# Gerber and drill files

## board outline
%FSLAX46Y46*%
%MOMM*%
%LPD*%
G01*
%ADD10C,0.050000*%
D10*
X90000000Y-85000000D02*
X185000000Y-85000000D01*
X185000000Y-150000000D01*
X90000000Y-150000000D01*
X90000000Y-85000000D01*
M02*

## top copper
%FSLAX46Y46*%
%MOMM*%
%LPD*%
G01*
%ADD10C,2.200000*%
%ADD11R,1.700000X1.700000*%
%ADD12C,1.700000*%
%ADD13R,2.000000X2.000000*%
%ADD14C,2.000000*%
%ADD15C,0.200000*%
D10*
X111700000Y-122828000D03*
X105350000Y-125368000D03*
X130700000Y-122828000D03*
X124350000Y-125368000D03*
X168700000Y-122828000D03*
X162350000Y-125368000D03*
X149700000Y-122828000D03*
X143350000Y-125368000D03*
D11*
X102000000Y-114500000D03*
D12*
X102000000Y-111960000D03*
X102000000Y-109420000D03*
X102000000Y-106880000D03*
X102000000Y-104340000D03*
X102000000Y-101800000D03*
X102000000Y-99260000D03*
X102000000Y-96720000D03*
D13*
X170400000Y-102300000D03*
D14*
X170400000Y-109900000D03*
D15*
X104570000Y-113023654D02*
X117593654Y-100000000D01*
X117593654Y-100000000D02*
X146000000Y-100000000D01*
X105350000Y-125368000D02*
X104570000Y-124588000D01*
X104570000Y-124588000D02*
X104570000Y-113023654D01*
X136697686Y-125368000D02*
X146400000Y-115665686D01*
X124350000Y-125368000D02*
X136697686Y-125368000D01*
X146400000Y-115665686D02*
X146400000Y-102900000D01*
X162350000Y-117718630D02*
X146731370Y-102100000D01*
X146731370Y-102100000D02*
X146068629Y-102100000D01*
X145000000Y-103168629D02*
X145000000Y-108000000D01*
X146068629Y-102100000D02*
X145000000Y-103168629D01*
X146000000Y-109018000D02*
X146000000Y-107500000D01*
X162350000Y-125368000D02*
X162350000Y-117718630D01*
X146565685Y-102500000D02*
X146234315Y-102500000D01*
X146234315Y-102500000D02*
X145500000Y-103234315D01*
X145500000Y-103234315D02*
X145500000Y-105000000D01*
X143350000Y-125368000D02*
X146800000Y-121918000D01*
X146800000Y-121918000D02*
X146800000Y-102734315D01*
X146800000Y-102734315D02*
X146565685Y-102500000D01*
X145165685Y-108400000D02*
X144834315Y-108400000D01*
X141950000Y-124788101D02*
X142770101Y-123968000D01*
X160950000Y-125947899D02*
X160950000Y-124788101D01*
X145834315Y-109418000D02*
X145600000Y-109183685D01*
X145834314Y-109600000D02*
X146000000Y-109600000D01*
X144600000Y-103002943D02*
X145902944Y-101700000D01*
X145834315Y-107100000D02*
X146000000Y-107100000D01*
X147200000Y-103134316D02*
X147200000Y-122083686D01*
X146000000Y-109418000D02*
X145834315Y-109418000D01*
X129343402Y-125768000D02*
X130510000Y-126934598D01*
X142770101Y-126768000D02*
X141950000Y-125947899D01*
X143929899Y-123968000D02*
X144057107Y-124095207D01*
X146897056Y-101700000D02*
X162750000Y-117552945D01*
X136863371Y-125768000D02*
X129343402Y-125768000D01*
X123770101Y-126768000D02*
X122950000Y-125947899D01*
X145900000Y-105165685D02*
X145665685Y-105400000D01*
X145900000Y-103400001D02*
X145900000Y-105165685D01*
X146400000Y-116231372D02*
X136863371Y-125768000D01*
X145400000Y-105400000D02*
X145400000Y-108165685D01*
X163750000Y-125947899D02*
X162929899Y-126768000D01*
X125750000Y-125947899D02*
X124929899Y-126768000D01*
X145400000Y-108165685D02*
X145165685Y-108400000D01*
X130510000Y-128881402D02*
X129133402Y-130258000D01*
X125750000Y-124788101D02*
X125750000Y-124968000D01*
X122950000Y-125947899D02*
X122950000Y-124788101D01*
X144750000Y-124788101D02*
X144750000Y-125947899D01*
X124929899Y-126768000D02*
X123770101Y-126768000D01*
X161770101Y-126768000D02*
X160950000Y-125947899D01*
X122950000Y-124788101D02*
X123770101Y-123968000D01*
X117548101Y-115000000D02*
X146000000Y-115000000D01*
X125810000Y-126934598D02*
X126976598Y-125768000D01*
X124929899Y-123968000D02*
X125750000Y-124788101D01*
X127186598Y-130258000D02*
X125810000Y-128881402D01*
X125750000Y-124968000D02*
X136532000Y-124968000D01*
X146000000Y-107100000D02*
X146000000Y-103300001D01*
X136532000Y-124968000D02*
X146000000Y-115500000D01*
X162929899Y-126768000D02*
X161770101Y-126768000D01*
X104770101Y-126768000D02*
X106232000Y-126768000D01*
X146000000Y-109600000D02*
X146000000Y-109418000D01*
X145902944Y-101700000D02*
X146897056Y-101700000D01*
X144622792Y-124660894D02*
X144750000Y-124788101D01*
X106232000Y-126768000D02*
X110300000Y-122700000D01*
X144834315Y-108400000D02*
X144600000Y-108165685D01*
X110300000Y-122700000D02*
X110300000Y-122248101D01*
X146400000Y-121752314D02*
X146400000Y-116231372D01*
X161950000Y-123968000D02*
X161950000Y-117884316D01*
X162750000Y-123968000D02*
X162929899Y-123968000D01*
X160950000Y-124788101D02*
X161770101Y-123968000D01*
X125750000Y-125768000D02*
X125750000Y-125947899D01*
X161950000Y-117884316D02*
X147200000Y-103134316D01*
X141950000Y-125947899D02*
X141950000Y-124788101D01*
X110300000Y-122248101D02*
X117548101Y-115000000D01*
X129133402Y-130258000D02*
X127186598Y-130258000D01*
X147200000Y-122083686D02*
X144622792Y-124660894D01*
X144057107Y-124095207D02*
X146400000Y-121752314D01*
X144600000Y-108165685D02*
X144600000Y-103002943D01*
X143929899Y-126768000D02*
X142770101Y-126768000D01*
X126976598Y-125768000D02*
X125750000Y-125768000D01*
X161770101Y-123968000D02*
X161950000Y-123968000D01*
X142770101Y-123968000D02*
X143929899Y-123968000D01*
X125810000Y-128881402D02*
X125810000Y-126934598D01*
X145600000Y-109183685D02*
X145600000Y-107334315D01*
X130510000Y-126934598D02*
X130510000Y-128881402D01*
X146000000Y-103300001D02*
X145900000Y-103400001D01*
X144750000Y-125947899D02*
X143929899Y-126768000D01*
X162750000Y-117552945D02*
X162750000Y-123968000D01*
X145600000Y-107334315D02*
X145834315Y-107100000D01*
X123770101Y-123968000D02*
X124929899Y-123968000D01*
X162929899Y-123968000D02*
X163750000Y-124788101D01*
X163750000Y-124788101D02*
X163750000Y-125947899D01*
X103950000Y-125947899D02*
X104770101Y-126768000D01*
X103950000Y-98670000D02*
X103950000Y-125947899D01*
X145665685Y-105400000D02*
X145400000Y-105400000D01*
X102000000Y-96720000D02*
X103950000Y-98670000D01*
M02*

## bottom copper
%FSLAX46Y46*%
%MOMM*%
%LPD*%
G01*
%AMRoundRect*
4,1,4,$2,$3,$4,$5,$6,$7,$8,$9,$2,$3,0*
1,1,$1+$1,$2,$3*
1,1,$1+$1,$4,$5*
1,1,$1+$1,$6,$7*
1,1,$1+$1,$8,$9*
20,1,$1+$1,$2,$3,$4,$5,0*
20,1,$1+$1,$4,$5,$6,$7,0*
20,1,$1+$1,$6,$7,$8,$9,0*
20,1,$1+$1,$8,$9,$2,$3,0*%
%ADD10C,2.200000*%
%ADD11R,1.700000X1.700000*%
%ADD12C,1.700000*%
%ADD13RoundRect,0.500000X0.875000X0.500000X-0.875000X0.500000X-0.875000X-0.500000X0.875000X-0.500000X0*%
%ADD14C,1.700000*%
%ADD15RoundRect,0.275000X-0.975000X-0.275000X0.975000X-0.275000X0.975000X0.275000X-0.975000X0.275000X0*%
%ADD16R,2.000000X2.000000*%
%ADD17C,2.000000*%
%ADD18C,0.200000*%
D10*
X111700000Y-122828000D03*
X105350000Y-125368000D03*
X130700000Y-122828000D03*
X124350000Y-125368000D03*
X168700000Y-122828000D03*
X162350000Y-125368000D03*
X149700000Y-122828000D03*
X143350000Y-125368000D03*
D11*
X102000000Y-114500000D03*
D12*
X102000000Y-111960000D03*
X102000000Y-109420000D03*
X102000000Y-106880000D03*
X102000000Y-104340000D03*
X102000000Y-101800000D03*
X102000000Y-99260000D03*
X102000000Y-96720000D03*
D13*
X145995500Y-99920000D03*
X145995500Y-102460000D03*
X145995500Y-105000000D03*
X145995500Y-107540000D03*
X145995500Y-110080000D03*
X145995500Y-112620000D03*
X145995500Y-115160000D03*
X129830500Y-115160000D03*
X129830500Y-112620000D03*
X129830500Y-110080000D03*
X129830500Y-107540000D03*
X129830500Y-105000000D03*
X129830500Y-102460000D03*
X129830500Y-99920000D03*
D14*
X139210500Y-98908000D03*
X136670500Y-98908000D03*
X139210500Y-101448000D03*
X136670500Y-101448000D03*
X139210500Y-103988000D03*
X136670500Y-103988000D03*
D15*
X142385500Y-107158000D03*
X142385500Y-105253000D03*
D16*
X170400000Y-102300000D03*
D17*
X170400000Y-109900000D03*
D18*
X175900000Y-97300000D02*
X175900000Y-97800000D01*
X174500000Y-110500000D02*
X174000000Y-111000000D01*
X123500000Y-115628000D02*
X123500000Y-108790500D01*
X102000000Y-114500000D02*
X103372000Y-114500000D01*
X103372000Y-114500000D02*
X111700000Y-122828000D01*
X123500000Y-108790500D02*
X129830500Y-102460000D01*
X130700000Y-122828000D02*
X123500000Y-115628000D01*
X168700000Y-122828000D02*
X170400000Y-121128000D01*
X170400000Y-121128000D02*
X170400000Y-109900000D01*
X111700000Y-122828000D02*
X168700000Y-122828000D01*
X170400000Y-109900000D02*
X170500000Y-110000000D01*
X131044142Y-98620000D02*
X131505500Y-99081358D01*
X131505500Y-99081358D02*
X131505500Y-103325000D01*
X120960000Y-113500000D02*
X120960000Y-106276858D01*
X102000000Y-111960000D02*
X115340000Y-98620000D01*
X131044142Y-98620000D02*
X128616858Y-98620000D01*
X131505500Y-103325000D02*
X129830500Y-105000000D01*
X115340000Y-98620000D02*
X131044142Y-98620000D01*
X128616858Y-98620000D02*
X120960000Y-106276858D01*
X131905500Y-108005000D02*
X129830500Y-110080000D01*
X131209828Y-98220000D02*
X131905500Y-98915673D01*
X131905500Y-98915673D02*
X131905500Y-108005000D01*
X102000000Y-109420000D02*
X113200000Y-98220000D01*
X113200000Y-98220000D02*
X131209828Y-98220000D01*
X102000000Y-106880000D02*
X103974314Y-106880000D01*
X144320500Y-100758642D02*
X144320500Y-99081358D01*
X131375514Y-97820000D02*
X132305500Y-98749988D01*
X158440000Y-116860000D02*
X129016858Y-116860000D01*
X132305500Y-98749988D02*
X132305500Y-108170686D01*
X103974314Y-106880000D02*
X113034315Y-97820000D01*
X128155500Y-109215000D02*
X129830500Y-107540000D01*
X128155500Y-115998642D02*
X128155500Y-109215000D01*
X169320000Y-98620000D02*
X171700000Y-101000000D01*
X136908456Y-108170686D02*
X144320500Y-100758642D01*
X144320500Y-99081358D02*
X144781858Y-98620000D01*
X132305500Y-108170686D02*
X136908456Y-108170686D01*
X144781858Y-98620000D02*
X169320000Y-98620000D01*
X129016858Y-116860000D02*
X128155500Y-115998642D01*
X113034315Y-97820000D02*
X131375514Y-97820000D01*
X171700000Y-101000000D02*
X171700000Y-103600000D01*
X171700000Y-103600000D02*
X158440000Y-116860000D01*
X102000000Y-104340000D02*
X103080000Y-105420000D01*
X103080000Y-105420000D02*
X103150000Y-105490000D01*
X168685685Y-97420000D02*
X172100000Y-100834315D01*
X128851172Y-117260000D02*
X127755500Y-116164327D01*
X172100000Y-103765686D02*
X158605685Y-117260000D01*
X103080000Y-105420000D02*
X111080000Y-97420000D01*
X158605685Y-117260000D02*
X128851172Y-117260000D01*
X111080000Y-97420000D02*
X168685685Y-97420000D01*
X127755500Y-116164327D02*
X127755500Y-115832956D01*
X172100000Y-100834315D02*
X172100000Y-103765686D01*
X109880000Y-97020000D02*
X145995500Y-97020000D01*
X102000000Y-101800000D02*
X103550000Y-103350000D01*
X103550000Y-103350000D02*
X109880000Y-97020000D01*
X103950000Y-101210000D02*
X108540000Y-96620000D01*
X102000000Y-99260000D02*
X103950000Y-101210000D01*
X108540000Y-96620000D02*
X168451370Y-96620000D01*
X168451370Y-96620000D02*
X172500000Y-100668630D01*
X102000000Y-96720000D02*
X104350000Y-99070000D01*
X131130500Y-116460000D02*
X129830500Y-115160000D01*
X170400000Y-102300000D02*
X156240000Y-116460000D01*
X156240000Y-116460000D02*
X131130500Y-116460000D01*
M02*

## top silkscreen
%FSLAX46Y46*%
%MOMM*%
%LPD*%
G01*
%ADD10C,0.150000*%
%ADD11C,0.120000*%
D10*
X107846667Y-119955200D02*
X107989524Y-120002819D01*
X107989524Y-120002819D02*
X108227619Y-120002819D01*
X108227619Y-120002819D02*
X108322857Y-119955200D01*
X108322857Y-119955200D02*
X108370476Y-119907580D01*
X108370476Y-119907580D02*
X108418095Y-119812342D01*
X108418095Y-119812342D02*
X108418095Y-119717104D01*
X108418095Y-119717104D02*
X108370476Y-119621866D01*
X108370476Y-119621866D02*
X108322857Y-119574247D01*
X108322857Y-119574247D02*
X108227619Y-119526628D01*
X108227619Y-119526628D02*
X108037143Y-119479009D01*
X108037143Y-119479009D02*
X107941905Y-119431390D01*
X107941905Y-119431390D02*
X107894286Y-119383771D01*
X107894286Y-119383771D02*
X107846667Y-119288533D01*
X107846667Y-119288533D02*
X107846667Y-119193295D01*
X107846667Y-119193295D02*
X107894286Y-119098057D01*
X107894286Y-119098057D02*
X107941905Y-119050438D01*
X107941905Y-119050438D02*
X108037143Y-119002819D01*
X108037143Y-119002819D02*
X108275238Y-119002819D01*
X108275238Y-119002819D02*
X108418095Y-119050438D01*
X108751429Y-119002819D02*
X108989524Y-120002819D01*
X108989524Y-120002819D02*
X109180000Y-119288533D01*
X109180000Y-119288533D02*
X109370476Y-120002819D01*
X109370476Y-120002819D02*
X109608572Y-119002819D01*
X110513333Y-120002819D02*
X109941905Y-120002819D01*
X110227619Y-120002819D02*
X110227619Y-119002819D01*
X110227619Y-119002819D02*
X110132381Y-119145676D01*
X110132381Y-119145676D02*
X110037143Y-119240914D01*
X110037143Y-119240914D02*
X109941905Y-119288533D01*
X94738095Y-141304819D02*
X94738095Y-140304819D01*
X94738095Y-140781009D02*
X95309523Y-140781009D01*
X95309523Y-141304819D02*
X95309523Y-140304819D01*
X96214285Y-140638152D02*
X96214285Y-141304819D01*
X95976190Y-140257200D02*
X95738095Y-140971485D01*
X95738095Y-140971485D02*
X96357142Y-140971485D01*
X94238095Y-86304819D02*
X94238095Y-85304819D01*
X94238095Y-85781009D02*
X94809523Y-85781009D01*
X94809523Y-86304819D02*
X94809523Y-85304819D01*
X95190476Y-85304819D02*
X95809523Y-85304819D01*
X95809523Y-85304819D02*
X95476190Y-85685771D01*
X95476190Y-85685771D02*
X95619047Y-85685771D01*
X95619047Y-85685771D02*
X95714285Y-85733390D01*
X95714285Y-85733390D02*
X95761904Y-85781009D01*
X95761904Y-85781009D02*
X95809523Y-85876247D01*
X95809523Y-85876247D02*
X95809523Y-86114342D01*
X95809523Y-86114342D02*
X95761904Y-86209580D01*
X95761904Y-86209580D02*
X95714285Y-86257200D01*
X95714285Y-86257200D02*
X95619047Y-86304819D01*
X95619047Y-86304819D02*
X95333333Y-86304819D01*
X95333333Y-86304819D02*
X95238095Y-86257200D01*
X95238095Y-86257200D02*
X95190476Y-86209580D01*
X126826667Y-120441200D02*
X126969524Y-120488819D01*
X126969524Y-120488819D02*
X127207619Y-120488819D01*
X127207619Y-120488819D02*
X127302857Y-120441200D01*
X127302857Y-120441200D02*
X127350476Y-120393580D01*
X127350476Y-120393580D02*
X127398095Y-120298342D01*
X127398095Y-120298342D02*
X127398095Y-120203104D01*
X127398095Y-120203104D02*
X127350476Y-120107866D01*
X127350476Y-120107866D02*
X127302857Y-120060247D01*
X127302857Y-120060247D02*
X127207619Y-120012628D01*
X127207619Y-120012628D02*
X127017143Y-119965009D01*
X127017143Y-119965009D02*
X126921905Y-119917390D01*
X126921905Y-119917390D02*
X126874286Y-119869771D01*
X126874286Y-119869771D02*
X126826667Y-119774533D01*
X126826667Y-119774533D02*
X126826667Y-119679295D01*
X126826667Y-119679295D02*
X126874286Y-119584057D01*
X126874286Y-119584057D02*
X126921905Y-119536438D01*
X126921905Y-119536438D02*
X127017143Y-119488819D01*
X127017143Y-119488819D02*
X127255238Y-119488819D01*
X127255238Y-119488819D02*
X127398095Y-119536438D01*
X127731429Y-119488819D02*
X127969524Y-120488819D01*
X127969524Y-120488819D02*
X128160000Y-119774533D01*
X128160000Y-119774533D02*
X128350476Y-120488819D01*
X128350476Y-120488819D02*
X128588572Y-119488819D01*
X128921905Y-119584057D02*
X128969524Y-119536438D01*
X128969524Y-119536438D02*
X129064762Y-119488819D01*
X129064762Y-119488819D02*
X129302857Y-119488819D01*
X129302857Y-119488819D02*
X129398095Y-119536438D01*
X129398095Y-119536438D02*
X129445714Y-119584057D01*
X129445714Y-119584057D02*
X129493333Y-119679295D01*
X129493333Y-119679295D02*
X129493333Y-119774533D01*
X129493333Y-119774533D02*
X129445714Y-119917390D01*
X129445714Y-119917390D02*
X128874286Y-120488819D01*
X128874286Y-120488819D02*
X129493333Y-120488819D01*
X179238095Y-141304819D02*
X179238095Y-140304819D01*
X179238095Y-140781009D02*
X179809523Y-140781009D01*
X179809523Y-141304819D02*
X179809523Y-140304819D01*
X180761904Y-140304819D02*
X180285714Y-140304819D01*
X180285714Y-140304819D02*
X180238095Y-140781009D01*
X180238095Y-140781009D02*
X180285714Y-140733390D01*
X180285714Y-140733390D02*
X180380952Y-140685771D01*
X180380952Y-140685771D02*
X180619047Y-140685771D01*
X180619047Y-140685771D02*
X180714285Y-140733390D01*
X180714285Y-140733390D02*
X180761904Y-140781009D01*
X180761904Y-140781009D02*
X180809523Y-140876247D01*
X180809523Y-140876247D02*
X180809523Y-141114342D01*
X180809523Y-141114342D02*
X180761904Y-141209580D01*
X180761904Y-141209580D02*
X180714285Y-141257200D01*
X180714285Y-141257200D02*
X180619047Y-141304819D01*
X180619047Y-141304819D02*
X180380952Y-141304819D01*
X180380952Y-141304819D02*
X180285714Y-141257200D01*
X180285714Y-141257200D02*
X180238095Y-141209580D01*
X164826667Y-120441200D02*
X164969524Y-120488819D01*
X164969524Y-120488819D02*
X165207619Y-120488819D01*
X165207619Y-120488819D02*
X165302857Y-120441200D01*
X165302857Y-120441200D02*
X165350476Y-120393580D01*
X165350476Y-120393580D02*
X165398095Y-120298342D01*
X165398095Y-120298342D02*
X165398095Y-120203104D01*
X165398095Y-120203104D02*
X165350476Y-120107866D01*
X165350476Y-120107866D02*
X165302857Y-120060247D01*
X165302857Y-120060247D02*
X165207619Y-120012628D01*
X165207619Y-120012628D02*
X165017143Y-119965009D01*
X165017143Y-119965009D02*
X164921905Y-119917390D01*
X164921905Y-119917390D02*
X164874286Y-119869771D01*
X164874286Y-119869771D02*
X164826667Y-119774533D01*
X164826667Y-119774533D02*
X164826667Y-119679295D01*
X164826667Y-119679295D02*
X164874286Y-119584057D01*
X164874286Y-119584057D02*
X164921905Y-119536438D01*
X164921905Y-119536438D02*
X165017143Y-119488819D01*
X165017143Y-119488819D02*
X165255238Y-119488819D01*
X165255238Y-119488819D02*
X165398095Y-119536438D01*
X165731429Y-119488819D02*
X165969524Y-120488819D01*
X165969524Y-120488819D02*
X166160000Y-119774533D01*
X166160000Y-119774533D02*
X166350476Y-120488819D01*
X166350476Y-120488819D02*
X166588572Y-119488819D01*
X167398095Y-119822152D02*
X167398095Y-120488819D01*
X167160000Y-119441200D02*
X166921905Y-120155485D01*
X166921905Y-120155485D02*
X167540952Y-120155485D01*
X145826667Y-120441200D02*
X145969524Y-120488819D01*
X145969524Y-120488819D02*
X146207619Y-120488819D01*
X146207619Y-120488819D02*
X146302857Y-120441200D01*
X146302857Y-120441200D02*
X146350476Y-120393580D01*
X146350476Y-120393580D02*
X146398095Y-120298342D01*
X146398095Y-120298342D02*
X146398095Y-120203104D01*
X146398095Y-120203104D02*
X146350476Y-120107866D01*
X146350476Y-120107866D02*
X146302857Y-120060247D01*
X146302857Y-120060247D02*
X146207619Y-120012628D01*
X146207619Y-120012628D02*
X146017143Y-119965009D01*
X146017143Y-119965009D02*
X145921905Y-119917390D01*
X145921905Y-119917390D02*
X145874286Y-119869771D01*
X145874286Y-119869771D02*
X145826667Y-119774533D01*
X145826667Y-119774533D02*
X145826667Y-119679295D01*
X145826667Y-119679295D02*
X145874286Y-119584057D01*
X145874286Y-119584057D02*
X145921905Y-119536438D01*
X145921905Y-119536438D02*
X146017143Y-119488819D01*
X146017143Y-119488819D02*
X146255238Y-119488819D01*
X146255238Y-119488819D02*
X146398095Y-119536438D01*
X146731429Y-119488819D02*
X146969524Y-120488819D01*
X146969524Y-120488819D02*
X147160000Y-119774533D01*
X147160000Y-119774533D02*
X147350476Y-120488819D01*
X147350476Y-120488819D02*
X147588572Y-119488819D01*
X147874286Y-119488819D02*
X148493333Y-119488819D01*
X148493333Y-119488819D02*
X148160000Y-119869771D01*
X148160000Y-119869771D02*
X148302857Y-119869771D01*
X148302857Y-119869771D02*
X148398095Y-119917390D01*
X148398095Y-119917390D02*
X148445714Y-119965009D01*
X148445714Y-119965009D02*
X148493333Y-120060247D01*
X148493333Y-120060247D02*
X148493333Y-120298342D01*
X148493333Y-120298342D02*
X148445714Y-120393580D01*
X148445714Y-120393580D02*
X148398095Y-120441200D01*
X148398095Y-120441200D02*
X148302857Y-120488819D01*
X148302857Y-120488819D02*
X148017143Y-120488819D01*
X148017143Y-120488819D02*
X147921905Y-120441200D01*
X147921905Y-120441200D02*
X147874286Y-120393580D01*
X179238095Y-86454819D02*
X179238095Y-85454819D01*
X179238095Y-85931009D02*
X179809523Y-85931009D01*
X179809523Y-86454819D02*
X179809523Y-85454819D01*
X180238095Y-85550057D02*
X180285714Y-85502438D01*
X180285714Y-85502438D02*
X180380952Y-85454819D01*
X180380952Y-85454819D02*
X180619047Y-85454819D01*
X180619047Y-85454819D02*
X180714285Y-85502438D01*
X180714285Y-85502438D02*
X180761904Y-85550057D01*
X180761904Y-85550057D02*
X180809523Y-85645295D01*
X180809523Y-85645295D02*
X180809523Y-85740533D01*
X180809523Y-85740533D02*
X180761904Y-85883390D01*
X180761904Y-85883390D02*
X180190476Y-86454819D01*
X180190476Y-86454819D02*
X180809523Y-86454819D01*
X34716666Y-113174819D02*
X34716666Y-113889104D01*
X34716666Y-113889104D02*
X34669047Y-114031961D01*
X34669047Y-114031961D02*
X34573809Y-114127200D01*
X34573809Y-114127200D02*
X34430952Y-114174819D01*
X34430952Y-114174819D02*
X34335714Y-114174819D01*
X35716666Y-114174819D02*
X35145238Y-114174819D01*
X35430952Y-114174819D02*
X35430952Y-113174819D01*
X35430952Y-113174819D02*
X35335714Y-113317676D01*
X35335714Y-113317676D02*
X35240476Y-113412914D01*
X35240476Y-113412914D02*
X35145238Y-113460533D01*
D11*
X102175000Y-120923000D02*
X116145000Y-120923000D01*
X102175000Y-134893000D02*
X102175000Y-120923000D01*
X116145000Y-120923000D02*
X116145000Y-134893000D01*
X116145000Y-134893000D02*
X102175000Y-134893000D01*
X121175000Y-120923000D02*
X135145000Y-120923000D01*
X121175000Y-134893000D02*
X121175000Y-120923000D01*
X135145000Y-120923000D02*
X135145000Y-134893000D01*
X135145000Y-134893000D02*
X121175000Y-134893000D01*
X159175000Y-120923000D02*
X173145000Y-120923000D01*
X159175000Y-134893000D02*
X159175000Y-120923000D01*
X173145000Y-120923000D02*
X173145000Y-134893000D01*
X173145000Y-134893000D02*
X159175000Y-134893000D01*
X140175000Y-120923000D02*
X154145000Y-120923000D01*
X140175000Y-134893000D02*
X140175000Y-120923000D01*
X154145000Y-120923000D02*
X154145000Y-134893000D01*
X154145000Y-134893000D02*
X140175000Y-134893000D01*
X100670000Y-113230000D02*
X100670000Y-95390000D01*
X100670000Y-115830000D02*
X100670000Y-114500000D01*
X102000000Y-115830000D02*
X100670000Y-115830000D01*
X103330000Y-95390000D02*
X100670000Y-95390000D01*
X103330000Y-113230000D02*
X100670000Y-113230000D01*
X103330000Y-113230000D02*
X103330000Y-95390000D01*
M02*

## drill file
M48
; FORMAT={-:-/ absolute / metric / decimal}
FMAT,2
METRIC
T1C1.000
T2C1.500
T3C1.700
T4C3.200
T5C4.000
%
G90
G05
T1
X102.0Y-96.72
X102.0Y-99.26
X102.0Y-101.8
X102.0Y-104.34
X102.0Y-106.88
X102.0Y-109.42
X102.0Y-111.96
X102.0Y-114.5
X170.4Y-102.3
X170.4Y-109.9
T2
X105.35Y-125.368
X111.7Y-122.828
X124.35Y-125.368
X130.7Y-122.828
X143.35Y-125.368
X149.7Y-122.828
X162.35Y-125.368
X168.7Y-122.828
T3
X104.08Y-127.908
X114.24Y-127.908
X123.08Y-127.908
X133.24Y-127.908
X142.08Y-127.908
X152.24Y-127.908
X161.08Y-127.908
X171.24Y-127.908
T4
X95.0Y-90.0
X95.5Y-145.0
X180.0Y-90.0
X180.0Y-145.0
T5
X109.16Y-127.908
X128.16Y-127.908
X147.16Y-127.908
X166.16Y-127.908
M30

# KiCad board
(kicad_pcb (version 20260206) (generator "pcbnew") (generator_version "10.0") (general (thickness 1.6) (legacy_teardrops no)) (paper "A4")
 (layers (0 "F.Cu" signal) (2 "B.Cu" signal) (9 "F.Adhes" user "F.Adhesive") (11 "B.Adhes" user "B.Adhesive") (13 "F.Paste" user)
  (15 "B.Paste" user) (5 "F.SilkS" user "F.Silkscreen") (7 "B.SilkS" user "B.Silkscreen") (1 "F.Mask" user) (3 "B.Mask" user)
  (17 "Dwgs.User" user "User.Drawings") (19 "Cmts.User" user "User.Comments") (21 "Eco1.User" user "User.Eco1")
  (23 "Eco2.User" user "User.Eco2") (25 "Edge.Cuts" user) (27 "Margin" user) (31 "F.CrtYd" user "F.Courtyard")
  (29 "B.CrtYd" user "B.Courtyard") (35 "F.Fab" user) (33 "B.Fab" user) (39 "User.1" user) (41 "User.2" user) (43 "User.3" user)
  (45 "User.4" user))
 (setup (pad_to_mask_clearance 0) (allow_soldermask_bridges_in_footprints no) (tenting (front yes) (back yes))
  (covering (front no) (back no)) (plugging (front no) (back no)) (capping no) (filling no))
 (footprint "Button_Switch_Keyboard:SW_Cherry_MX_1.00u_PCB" (layer "F.Cu") (at 111.7 122.828)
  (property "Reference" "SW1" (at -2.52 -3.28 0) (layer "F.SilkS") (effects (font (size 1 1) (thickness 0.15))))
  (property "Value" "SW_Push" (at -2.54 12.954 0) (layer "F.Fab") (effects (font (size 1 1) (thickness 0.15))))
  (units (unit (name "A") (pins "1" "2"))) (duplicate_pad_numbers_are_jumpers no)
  (fp_line (start -9.525 -1.905) (end 4.445 -1.905) (stroke (width 0.12) (type solid)) (layer "F.SilkS"))
  (fp_line (start -9.525 12.065) (end -9.525 -1.905) (stroke (width 0.12) (type solid)) (layer "F.SilkS"))
  (fp_line (start 4.445 -1.905) (end 4.445 12.065) (stroke (width 0.12) (type solid)) (layer "F.SilkS"))
  (fp_line (start 4.445 12.065) (end -9.525 12.065) (stroke (width 0.12) (type solid)) (layer "F.SilkS"))
  (pad "" np_thru_hole circle (at -7.62 5.08) (size 1.7 1.7) (drill 1.7) (layers "*.Cu" "*.Mask"))
  (pad "" np_thru_hole circle (at -2.54 5.08) (size 4 4) (drill 4) (layers "*.Cu" "*.Mask"))
  (pad "" np_thru_hole circle (at 2.54 5.08) (size 1.7 1.7) (drill 1.7) (layers "*.Cu" "*.Mask"))
  (pad "1" thru_hole circle (at 0 0) (size 2.2 2.2) (drill 1.5) (layers "*.Cu" "*.Mask") (remove_unused_layers no) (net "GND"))
  (pad "2" thru_hole circle (at -6.35 2.54) (size 2.2 2.2) (drill 1.5) (layers "*.Cu" "*.Mask") (remove_unused_layers no)
   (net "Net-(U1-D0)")))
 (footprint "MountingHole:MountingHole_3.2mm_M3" (layer "F.Cu") (at 95.5 145)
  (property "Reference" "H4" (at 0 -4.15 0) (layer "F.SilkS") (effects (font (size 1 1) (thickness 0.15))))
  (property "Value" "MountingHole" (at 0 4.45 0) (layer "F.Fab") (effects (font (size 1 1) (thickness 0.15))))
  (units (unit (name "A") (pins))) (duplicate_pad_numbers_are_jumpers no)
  (pad "" np_thru_hole circle (at 0 0) (size 3.2 3.2) (drill 3.2) (layers "*.Cu" "*.Mask")))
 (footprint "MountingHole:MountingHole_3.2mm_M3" (layer "F.Cu") (at 95 90)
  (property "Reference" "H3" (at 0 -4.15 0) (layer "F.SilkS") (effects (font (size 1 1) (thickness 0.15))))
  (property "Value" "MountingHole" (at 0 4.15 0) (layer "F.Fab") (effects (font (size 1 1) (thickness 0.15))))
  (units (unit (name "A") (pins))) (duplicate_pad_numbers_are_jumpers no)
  (pad "" np_thru_hole circle (at 0 0) (size 3.2 3.2) (drill 3.2) (layers "*.Cu" "*.Mask")))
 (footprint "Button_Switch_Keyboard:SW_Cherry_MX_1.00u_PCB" (layer "F.Cu") (at 130.7 122.828)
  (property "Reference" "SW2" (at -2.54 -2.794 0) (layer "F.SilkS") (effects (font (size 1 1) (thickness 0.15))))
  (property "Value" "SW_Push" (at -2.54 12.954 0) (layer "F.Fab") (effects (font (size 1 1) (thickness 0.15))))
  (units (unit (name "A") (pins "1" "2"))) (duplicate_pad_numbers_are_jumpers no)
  (fp_line (start -9.525 -1.905) (end 4.445 -1.905) (stroke (width 0.12) (type solid)) (layer "F.SilkS"))
  (fp_line (start -9.525 12.065) (end -9.525 -1.905) (stroke (width 0.12) (type solid)) (layer "F.SilkS"))
  (fp_line (start 4.445 -1.905) (end 4.445 12.065) (stroke (width 0.12) (type solid)) (layer "F.SilkS"))
  (fp_line (start 4.445 12.065) (end -9.525 12.065) (stroke (width 0.12) (type solid)) (layer "F.SilkS"))
  (pad "" np_thru_hole circle (at -7.62 5.08) (size 1.7 1.7) (drill 1.7) (layers "*.Cu" "*.Mask"))
  (pad "" np_thru_hole circle (at -2.54 5.08) (size 4 4) (drill 4) (layers "*.Cu" "*.Mask"))
  (pad "" np_thru_hole circle (at 2.54 5.08) (size 1.7 1.7) (drill 1.7) (layers "*.Cu" "*.Mask"))
  (pad "1" thru_hole circle (at 0 0) (size 2.2 2.2) (drill 1.5) (layers "*.Cu" "*.Mask") (remove_unused_layers no) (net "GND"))
  (pad "2" thru_hole circle (at -6.35 2.54) (size 2.2 2.2) (drill 1.5) (layers "*.Cu" "*.Mask") (remove_unused_layers no)
   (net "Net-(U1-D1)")))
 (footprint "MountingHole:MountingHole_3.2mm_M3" (layer "F.Cu") (at 180 145)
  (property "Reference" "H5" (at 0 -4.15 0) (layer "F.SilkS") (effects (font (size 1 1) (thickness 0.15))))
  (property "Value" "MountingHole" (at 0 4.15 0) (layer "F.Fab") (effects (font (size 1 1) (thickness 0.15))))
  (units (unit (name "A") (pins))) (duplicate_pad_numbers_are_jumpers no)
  (pad "" np_thru_hole circle (at 0 0) (size 3.2 3.2) (drill 3.2) (layers "*.Cu" "*.Mask")))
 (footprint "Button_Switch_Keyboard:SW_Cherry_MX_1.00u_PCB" (layer "F.Cu") (at 168.7 122.828)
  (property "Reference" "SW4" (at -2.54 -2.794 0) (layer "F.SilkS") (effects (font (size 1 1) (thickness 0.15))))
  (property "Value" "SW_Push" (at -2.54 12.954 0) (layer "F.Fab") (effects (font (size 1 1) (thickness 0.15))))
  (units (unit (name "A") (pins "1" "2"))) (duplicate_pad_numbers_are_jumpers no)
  (fp_line (start -9.525 -1.905) (end 4.445 -1.905) (stroke (width 0.12) (type solid)) (layer "F.SilkS"))
  (fp_line (start -9.525 12.065) (end -9.525 -1.905) (stroke (width 0.12) (type solid)) (layer "F.SilkS"))
  (fp_line (start 4.445 -1.905) (end 4.445 12.065) (stroke (width 0.12) (type solid)) (layer "F.SilkS"))
  (fp_line (start 4.445 12.065) (end -9.525 12.065) (stroke (width 0.12) (type solid)) (layer "F.SilkS"))
  (pad "" np_thru_hole circle (at -7.62 5.08) (size 1.7 1.7) (drill 1.7) (layers "*.Cu" "*.Mask"))
  (pad "" np_thru_hole circle (at -2.54 5.08) (size 4 4) (drill 4) (layers "*.Cu" "*.Mask"))
  (pad "" np_thru_hole circle (at 2.54 5.08) (size 1.7 1.7) (drill 1.7) (layers "*.Cu" "*.Mask"))
  (pad "1" thru_hole circle (at 0 0) (size 2.2 2.2) (drill 1.5) (layers "*.Cu" "*.Mask") (remove_unused_layers no) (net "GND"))
  (pad "2" thru_hole circle (at -6.35 2.54) (size 2.2 2.2) (drill 1.5) (layers "*.Cu" "*.Mask") (remove_unused_layers no)
   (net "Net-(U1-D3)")))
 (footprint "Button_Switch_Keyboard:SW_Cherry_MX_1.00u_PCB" (layer "F.Cu") (at 149.7 122.828)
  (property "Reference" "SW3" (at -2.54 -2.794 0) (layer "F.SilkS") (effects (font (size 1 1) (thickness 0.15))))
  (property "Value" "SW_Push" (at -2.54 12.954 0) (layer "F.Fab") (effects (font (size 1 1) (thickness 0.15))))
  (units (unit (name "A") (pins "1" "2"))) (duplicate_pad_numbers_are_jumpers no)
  (fp_line (start -9.525 -1.905) (end 4.445 -1.905) (stroke (width 0.12) (type solid)) (layer "F.SilkS"))
  (fp_line (start -9.525 12.065) (end -9.525 -1.905) (stroke (width 0.12) (type solid)) (layer "F.SilkS"))
  (fp_line (start 4.445 -1.905) (end 4.445 12.065) (stroke (width 0.12) (type solid)) (layer "F.SilkS"))
  (fp_line (start 4.445 12.065) (end -9.525 12.065) (stroke (width 0.12) (type solid)) (layer "F.SilkS"))
  (pad "" np_thru_hole circle (at -7.62 5.08) (size 1.7 1.7) (drill 1.7) (layers "*.Cu" "*.Mask"))
  (pad "" np_thru_hole circle (at -2.54 5.08) (size 4 4) (drill 4) (layers "*.Cu" "*.Mask"))
  (pad "" np_thru_hole circle (at 2.54 5.08) (size 1.7 1.7) (drill 1.7) (layers "*.Cu" "*.Mask"))
  (pad "1" thru_hole circle (at 0 0) (size 2.2 2.2) (drill 1.5) (layers "*.Cu" "*.Mask") (remove_unused_layers no) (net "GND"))
  (pad "2" thru_hole circle (at -6.35 2.54) (size 2.2 2.2) (drill 1.5) (layers "*.Cu" "*.Mask") (remove_unused_layers no)
   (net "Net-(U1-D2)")))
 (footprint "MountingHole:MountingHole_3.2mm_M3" (layer "F.Cu") (at 180 90)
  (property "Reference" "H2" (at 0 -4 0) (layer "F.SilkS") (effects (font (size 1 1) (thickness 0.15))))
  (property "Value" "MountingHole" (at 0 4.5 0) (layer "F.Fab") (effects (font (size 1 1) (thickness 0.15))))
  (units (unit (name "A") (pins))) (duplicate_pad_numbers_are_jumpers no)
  (pad "" np_thru_hole circle (at 0 0) (size 3.2 3.2) (drill 3.2) (layers "*.Cu" "*.Mask")))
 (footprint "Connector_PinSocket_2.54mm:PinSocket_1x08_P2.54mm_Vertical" (layer "F.Cu") (at 102 114.5 180)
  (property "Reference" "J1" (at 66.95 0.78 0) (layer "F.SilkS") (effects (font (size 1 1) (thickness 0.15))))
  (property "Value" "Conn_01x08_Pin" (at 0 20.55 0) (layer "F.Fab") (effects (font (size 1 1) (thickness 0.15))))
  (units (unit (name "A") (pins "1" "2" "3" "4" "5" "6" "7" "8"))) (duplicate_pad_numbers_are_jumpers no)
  (fp_line (start 1.33 1.27) (end 1.33 19.11) (stroke (width 0.12) (type solid)) (layer "F.SilkS"))
  (fp_line (start 1.33 -1.33) (end 1.33 0) (stroke (width 0.12) (type solid)) (layer "F.SilkS"))
  (fp_line (start 0 -1.33) (end 1.33 -1.33) (stroke (width 0.12) (type solid)) (layer "F.SilkS"))
  (fp_line (start -1.33 19.11) (end 1.33 19.11) (stroke (width 0.12) (type solid)) (layer "F.SilkS"))
  (fp_line (start -1.33 1.27) (end 1.33 1.27) (stroke (width 0.12) (type solid)) (layer "F.SilkS"))
  (fp_line (start -1.33 1.27) (end -1.33 19.11) (stroke (width 0.12) (type solid)) (layer "F.SilkS"))
  (pad "1" thru_hole rect (at 0 0 180) (size 1.7 1.7) (drill 1) (layers "*.Cu" "*.Mask") (remove_unused_layers no) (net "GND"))
  (pad "2" thru_hole circle (at 0 2.54 180) (size 1.7 1.7) (drill 1) (layers "*.Cu" "*.Mask") (remove_unused_layers no) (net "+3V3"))
  (pad "3" thru_hole circle (at 0 5.08 180) (size 1.7 1.7) (drill 1) (layers "*.Cu" "*.Mask") (remove_unused_layers no) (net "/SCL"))
  (pad "4" thru_hole circle (at 0 7.62 180) (size 1.7 1.7) (drill 1) (layers "*.Cu" "*.Mask") (remove_unused_layers no) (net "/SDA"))
  (pad "5" thru_hole circle (at 0 10.16 180) (size 1.7 1.7) (drill 1) (layers "*.Cu" "*.Mask") (remove_unused_layers no) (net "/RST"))
  (pad "6" thru_hole circle (at 0 12.7 180) (size 1.7 1.7) (drill 1) (layers "*.Cu" "*.Mask") (remove_unused_layers no) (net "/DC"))
  (pad "7" thru_hole circle (at 0 15.24 180) (size 1.7 1.7) (drill 1) (layers "*.Cu" "*.Mask") (remove_unused_layers no) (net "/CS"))
  (pad "8" thru_hole circle (at 0 17.78 180) (size 1.7 1.7) (drill 1) (layers "*.Cu" "*.Mask") (remove_unused_layers no) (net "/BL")))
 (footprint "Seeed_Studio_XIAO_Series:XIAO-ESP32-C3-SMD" (layer "B.Cu") (at 146.8305 118.04 180)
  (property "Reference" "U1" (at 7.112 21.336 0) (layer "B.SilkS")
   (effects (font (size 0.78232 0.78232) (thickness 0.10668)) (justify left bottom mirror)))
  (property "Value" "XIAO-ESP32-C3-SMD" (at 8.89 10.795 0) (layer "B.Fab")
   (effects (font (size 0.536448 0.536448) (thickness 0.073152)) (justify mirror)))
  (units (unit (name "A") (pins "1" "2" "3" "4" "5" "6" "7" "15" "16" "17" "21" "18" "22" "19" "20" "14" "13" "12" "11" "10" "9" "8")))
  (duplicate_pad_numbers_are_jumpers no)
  (pad "1" smd roundrect (at 0.835 18.12 180) (size 2.75 2) (layers "B.Cu" "B.Mask" "B.Paste") (roundrect_rratio 0.25) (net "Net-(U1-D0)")
   (solder_mask_margin 0.0508) (thermal_bridge_angle 45))
  (pad "2" smd roundrect (at 0.835 15.58 180) (size 2.75 2) (layers "B.Cu" "B.Mask" "B.Paste") (roundrect_rratio 0.25) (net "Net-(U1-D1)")
   (solder_mask_margin 0.0508) (thermal_bridge_angle 45))
  (pad "3" smd roundrect (at 0.835 13.04 180) (size 2.75 2) (layers "B.Cu" "B.Mask" "B.Paste") (roundrect_rratio 0.25) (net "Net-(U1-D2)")
   (solder_mask_margin 0.0508) (thermal_bridge_angle 45))
  (pad "4" smd roundrect (at 0.835 10.5 180) (size 2.75 2) (layers "B.Cu" "B.Mask" "B.Paste") (roundrect_rratio 0.25) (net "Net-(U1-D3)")
   (solder_mask_margin 0.0508) (thermal_bridge_angle 45))
  (pad "5" smd roundrect (at 0.835 7.96 180) (size 2.75 2) (layers "B.Cu" "B.Mask" "B.Paste") (roundrect_rratio 0.25) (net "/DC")
   (solder_mask_margin 0.0508) (thermal_bridge_angle 45))
  (pad "6" smd roundrect (at 0.835 5.42 180) (size 2.75 2) (layers "B.Cu" "B.Mask" "B.Paste") (roundrect_rratio 0.25) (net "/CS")
   (solder_mask_margin 0.0508) (thermal_bridge_angle 45))
  (pad "7" smd roundrect (at 0.835 2.88 180) (size 2.75 2) (layers "B.Cu" "B.Mask" "B.Paste") (roundrect_rratio 0.25) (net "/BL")
   (solder_mask_margin 0.0508) (thermal_bridge_angle 45))
  (pad "8" smd roundrect (at 17 2.88 180) (size 2.75 2) (layers "B.Cu" "B.Mask" "B.Paste") (roundrect_rratio 0.25) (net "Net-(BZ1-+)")
   (solder_mask_margin 0.0508) (thermal_bridge_angle 45))
  (pad "9" smd roundrect (at 17 5.42 180) (size 2.75 2) (layers "B.Cu" "B.Mask" "B.Paste") (roundrect_rratio 0.25) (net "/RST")
   (solder_mask_margin 0.0508) (thermal_bridge_angle 45))
  (pad "10" smd roundrect (at 17 7.96 180) (size 2.75 2) (layers "B.Cu" "B.Mask" "B.Paste") (roundrect_rratio 0.25) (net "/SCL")
   (solder_mask_margin 0.0508) (thermal_bridge_angle 45))
  (pad "11" smd roundrect (at 17 10.5 180) (size 2.75 2) (layers "B.Cu" "B.Mask" "B.Paste") (roundrect_rratio 0.25) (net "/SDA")
   (solder_mask_margin 0.0508) (thermal_bridge_angle 45))
  (pad "12" smd roundrect (at 17 13.04 180) (size 2.75 2) (layers "B.Cu" "B.Mask" "B.Paste") (roundrect_rratio 0.25) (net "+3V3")
   (solder_mask_margin 0.0508) (thermal_bridge_angle 45))
  (pad "13" smd roundrect (at 17 15.58 180) (size 2.75 2) (layers "B.Cu" "B.Mask" "B.Paste") (roundrect_rratio 0.25) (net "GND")
   (solder_mask_margin 0.0508) (thermal_bridge_angle 45))
  (pad "14" smd roundrect (at 17 18.12 180) (size 2.75 2) (layers "B.Cu" "B.Mask" "B.Paste") (roundrect_rratio 0.25)
   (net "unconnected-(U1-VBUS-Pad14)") (solder_mask_margin 0.0508) (thermal_bridge_angle 45))
  (pad "15" smd circle (at 7.62 19.132 180) (size 1.7 1.7) (layers "B.Cu" "B.Mask" "B.Paste") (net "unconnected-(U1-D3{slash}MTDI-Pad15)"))
  (pad "16" smd circle (at 10.16 19.132 180) (size 1.7 1.7) (layers "B.Cu" "B.Mask" "B.Paste") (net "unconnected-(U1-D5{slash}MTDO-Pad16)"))
  (pad "17" smd circle (at 7.62 16.592 180) (size 1.7 1.7) (layers "B.Cu" "B.Mask" "B.Paste") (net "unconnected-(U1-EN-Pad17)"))
  (pad "18" smd circle (at 10.16 16.592 180) (size 1.7 1.7) (layers "B.Cu" "B.Mask" "B.Paste") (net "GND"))
  (pad "19" smd circle (at 7.62 14.052 180) (size 1.7 1.7) (layers "B.Cu" "B.Mask" "B.Paste") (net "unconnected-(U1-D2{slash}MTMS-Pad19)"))
  (pad "20" smd circle (at 10.16 14.052 180) (size 1.7 1.7) (layers "B.Cu" "B.Mask" "B.Paste") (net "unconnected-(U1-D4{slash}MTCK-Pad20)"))
  (pad "21" smd roundrect (at 4.445 10.882) (size 2.5 1.1) (layers "B.Cu" "B.Mask" "B.Paste") (roundrect_rratio 0.25)
   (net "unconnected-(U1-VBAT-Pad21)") (thermal_bridge_angle 45))
  (pad "22" smd roundrect (at 4.445 12.787) (size 2.5 1.1) (layers "B.Cu" "B.Mask" "B.Paste") (roundrect_rratio 0.25) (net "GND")
   (thermal_bridge_angle 45)))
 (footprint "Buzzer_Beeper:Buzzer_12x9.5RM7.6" (layer "B.Cu") (at 170.4 102.3 -90)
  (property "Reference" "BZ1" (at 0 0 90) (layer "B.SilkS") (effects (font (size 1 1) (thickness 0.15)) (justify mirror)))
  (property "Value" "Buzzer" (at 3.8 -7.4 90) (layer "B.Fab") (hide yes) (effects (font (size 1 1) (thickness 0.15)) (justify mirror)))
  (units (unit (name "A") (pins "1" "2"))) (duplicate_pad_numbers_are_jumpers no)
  (pad "1" thru_hole rect (at 0 0 270) (size 2 2) (drill 1) (layers "*.Cu" "*.Mask") (remove_unused_layers no) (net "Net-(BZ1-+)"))
  (pad "2" thru_hole circle (at 7.6 0 270) (size 2 2) (drill 1) (layers "*.Cu" "*.Mask") (remove_unused_layers no) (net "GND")))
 (gr_rect (start 90 85) (end 185 150) (stroke (width 0.05) (type default)) (fill no) (layer "Edge.Cuts"))
 (segment (start 175.9 97.3) (end 175.9 97.8) (width 0.2) (layer "B.Cu") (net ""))
 (segment (start 174.5 110.5) (end 174 111) (width 0.2) (layer "B.Cu") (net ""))
 (segment (start 123.5 115.628) (end 123.5 108.7905) (width 0.2) (layer "B.Cu") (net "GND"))
 (segment (start 102 114.5) (end 103.372 114.5) (width 0.2) (layer "B.Cu") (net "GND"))
 (segment (start 103.372 114.5) (end 111.7 122.828) (width 0.2) (layer "B.Cu") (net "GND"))
 (segment (start 123.5 108.7905) (end 129.8305 102.46) (width 0.2) (layer "B.Cu") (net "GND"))
 (segment (start 130.7 122.828) (end 123.5 115.628) (width 0.2) (layer "B.Cu") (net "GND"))
 (segment (start 168.7 122.828) (end 170.4 121.128) (width 0.2) (layer "B.Cu") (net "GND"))
 (segment (start 170.4 121.128) (end 170.4 109.9) (width 0.2) (layer "B.Cu") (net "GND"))
 (segment (start 111.7 122.828) (end 168.7 122.828) (width 0.2) (layer "B.Cu") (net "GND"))
 (segment (start 170.4 109.9) (end 170.5 110) (width 0.2) (layer "B.Cu") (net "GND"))
 (segment (start 104.57 113.023654) (end 117.593654 100) (width 0.2) (layer "F.Cu") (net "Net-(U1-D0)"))
 (segment (start 117.593654 100) (end 146 100) (width 0.2) (layer "F.Cu") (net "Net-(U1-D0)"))
 (segment (start 105.35 125.368) (end 104.57 124.588) (width 0.2) (layer "F.Cu") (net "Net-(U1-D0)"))
 (segment (start 104.57 124.588) (end 104.57 113.023654) (width 0.2) (layer "F.Cu") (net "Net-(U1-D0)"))
 (segment (start 136.697686 125.368) (end 146.4 115.665686) (width 0.2) (layer "F.Cu") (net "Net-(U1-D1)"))
 (segment (start 124.35 125.368) (end 136.697686 125.368) (width 0.2) (layer "F.Cu") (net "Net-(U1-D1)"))
 (segment (start 146.4 115.665686) (end 146.4 102.9) (width 0.2) (layer "F.Cu") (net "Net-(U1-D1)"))
 (segment (start 162.35 117.71863) (end 146.73137 102.1) (width 0.2) (layer "F.Cu") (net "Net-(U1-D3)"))
 (segment (start 146.73137 102.1) (end 146.068629 102.1) (width 0.2) (layer "F.Cu") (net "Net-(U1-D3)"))
 (segment (start 145 103.168629) (end 145 108) (width 0.2) (layer "F.Cu") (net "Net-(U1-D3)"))
 (segment (start 146.068629 102.1) (end 145 103.168629) (width 0.2) (layer "F.Cu") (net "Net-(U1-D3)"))
 (segment (start 146 109.018) (end 146 107.5) (width 0.2) (layer "F.Cu") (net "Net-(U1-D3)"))
 (segment (start 162.35 125.368) (end 162.35 117.71863) (width 0.2) (layer "F.Cu") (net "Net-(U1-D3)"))
 (segment (start 146.565685 102.5) (end 146.234315 102.5) (width 0.2) (layer "F.Cu") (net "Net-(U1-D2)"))
 (segment (start 146.234315 102.5) (end 145.5 103.234315) (width 0.2) (layer "F.Cu") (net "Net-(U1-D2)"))
 (segment (start 145.5 103.234315) (end 145.5 105) (width 0.2) (layer "F.Cu") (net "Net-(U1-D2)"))
 (segment (start 143.35 125.368) (end 146.8 121.918) (width 0.2) (layer "F.Cu") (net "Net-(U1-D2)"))
 (segment (start 146.8 121.918) (end 146.8 102.734315) (width 0.2) (layer "F.Cu") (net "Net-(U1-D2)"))
 (segment (start 146.8 102.734315) (end 146.565685 102.5) (width 0.2) (layer "F.Cu") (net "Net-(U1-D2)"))
 (segment (start 131.044142 98.62) (end 131.5055 99.081358) (width 0.2) (layer "B.Cu") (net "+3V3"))
 (segment (start 131.5055 99.081358) (end 131.5055 103.325) (width 0.2) (layer "B.Cu") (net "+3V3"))
 (segment (start 120.96 113.5) (end 120.96 106.276858) (width 0.2) (layer "B.Cu") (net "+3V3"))
 (segment (start 102 111.96) (end 115.34 98.62) (width 0.2) (layer "B.Cu") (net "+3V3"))
 (segment (start 131.044142 98.62) (end 128.616858 98.62) (width 0.2) (layer "B.Cu") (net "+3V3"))
 (segment (start 131.5055 103.325) (end 129.8305 105) (width 0.2) (layer "B.Cu") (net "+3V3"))
 (segment (start 115.34 98.62) (end 131.044142 98.62) (width 0.2) (layer "B.Cu") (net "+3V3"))
 (segment (start 128.616858 98.62) (end 120.96 106.276858) (width 0.2) (layer "B.Cu") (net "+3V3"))
 (segment (start 131.9055 108.005) (end 129.8305 110.08) (width 0.2) (layer "B.Cu") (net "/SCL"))
 (segment (start 131.209828 98.22) (end 131.9055 98.915673) (width 0.2) (layer "B.Cu") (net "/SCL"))
 (segment (start 131.9055 98.915673) (end 131.9055 108.005) (width 0.2) (layer "B.Cu") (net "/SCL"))
 (segment (start 102 109.42) (end 113.2 98.22) (width 0.2) (layer "B.Cu") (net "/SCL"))
 (segment (start 113.2 98.22) (end 131.209828 98.22) (width 0.2) (layer "B.Cu") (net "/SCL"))
 (segment (start 102 106.88) (end 103.974314 106.88) (width 0.2) (layer "B.Cu") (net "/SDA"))
 (segment (start 144.3205 100.758642) (end 144.3205 99.081358) (width 0.2) (layer "B.Cu") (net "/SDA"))
 (segment (start 131.375514 97.82) (end 132.3055 98.749988) (width 0.2) (layer "B.Cu") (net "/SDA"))
 (segment (start 158.44 116.86) (end 129.016858 116.86) (width 0.2) (layer "B.Cu") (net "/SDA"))
 (segment (start 132.3055 98.749988) (end 132.3055 108.170686) (width 0.2) (layer "B.Cu") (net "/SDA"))
 (segment (start 103.974314 106.88) (end 113.034315 97.82) (width 0.2) (layer "B.Cu") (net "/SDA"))
 (segment (start 128.1555 109.215) (end 129.8305 107.54) (width 0.2) (layer "B.Cu") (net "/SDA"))
 (segment (start 128.1555 115.998642) (end 128.1555 109.215) (width 0.2) (layer "B.Cu") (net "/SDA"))
 (segment (start 169.32 98.62) (end 171.7 101) (width 0.2) (layer "B.Cu") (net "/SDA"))
 (segment (start 136.908456 108.170686) (end 144.3205 100.758642) (width 0.2) (layer "B.Cu") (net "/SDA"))
 (segment (start 144.3205 99.081358) (end 144.781858 98.62) (width 0.2) (layer "B.Cu") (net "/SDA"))
 (segment (start 132.3055 108.170686) (end 136.908456 108.170686) (width 0.2) (layer "B.Cu") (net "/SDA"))
 (segment (start 144.781858 98.62) (end 169.32 98.62) (width 0.2) (layer "B.Cu") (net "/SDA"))
 (segment (start 129.016858 116.86) (end 128.1555 115.998642) (width 0.2) (layer "B.Cu") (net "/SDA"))
 (segment (start 113.034315 97.82) (end 131.375514 97.82) (width 0.2) (layer "B.Cu") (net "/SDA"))
 (segment (start 171.7 101) (end 171.7 103.6) (width 0.2) (layer "B.Cu") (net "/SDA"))
 (segment (start 171.7 103.6) (end 158.44 116.86) (width 0.2) (layer "B.Cu") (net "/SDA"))
 (segment (start 102 104.34) (end 103.08 105.42) (width 0.2) (layer "B.Cu") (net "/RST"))
 (segment (start 103.08 105.42) (end 103.15 105.49) (width 0.2) (layer "B.Cu") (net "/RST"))
 (segment (start 168.685685 97.42) (end 172.1 100.834315) (width 0.2) (layer "B.Cu") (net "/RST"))
 (segment (start 128.851172 117.26) (end 127.7555 116.164327) (width 0.2) (layer "B.Cu") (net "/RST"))
 (segment (start 172.1 103.765686) (end 158.605685 117.26) (width 0.2) (layer "B.Cu") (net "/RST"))
 (segment (start 103.08 105.42) (end 111.08 97.42) (width 0.2) (layer "B.Cu") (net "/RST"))
 (segment (start 158.605685 117.26) (end 128.851172 117.26) (width 0.2) (layer "B.Cu") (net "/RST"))
 (segment (start 111.08 97.42) (end 168.685685 97.42) (width 0.2) (layer "B.Cu") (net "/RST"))
 (segment (start 127.7555 116.164327) (end 127.7555 115.832956) (width 0.2) (layer "B.Cu") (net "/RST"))
 (segment (start 172.1 100.834315) (end 172.1 103.765686) (width 0.2) (layer "B.Cu") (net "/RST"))
 (segment (start 109.88 97.02) (end 145.9955 97.02) (width 0.2) (layer "B.Cu") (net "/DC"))
 (segment (start 102 101.8) (end 103.55 103.35) (width 0.2) (layer "B.Cu") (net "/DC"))
 (segment (start 103.55 103.35) (end 109.88 97.02) (width 0.2) (layer "B.Cu") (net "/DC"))
 (segment (start 103.95 101.21) (end 108.54 96.62) (width 0.2) (layer "B.Cu") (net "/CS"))
 (segment (start 102 99.26) (end 103.95 101.21) (width 0.2) (layer "B.Cu") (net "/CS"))
 (segment (start 108.54 96.62) (end 168.45137 96.62) (width 0.2) (layer "B.Cu") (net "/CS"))
 (segment (start 168.45137 96.62) (end 172.5 100.66863) (width 0.2) (layer "B.Cu") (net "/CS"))
 (segment (start 145.165685 108.4) (end 144.834315 108.4) (width 0.2) (layer "F.Cu") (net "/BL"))
 (segment (start 141.95 124.788101) (end 142.770101 123.968) (width 0.2) (layer "F.Cu") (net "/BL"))
 (segment (start 160.95 125.947899) (end 160.95 124.788101) (width 0.2) (layer "F.Cu") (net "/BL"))
 (segment (start 145.834315 109.418) (end 145.6 109.183685) (width 0.2) (layer "F.Cu") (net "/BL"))
 (segment (start 145.834314 109.6) (end 146 109.6) (width 0.2) (layer "F.Cu") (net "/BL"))
 (segment (start 144.6 103.002943) (end 145.902944 101.7) (width 0.2) (layer "F.Cu") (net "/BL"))
 (segment (start 145.834315 107.1) (end 146 107.1) (width 0.2) (layer "F.Cu") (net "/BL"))
 (segment (start 147.2 103.134316) (end 147.2 122.083686) (width 0.2) (layer "F.Cu") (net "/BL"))
 (segment (start 146 109.418) (end 145.834315 109.418) (width 0.2) (layer "F.Cu") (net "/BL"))
 (segment (start 129.343402 125.768) (end 130.51 126.934598) (width 0.2) (layer "F.Cu") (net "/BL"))
 (segment (start 142.770101 126.768) (end 141.95 125.947899) (width 0.2) (layer "F.Cu") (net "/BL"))
 (segment (start 143.929899 123.968) (end 144.057107 124.095207) (width 0.2) (layer "F.Cu") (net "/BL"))
 (segment (start 146.897056 101.7) (end 162.75 117.552945) (width 0.2) (layer "F.Cu") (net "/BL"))
 (segment (start 136.863371 125.768) (end 129.343402 125.768) (width 0.2) (layer "F.Cu") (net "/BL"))
 (segment (start 123.770101 126.768) (end 122.95 125.947899) (width 0.2) (layer "F.Cu") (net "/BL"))
 (segment (start 145.9 105.165685) (end 145.665685 105.4) (width 0.2) (layer "F.Cu") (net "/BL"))
 (segment (start 145.9 103.400001) (end 145.9 105.165685) (width 0.2) (layer "F.Cu") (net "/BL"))
 (segment (start 146.4 116.231372) (end 136.863371 125.768) (width 0.2) (layer "F.Cu") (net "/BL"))
 (segment (start 145.4 105.4) (end 145.4 108.165685) (width 0.2) (layer "F.Cu") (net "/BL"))
 (segment (start 163.75 125.947899) (end 162.929899 126.768) (width 0.2) (layer "F.Cu") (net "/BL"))
 (segment (start 125.75 125.947899) (end 124.929899 126.768) (width 0.2) (layer "F.Cu") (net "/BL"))
 (segment (start 145.4 108.165685) (end 145.165685 108.4) (width 0.2) (layer "F.Cu") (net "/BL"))
 (segment (start 130.51 128.881402) (end 129.133402 130.258) (width 0.2) (layer "F.Cu") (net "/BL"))
 (segment (start 125.75 124.788101) (end 125.75 124.968) (width 0.2) (layer "F.Cu") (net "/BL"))
 (segment (start 122.95 125.947899) (end 122.95 124.788101) (width 0.2) (layer "F.Cu") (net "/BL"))
 (segment (start 144.75 124.788101) (end 144.75 125.947899) (width 0.2) (layer "F.Cu") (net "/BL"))
 (segment (start 124.929899 126.768) (end 123.770101 126.768) (width 0.2) (layer "F.Cu") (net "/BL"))
 (segment (start 161.770101 126.768) (end 160.95 125.947899) (width 0.2) (layer "F.Cu") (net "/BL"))
 (segment (start 122.95 124.788101) (end 123.770101 123.968) (width 0.2) (layer "F.Cu") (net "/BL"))
 (segment (start 117.548101 115) (end 146 115) (width 0.2) (layer "F.Cu") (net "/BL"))
 (segment (start 125.81 126.934598) (end 126.976598 125.768) (width 0.2) (layer "F.Cu") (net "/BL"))
 (segment (start 124.929899 123.968) (end 125.75 124.788101) (width 0.2) (layer "F.Cu") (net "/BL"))
 (segment (start 127.186598 130.258) (end 125.81 128.881402) (width 0.2) (layer "F.Cu") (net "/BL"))
 (segment (start 125.75 124.968) (end 136.532 124.968) (width 0.2) (layer "F.Cu") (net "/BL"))
 (segment (start 146 107.1) (end 146 103.300001) (width 0.2) (layer "F.Cu") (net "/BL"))
 (segment (start 136.532 124.968) (end 146 115.5) (width 0.2) (layer "F.Cu") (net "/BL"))
 (segment (start 162.929899 126.768) (end 161.770101 126.768) (width 0.2) (layer "F.Cu") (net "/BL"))
 (segment (start 104.770101 126.768) (end 106.232 126.768) (width 0.2) (layer "F.Cu") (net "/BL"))
 (segment (start 146 109.6) (end 146 109.418) (width 0.2) (layer "F.Cu") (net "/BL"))
 (segment (start 145.902944 101.7) (end 146.897056 101.7) (width 0.2) (layer "F.Cu") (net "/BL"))
 (segment (start 144.622792 124.660894) (end 144.75 124.788101) (width 0.2) (layer "F.Cu") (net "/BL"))
 (segment (start 106.232 126.768) (end 110.3 122.7) (width 0.2) (layer "F.Cu") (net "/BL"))
 (segment (start 144.834315 108.4) (end 144.6 108.165685) (width 0.2) (layer "F.Cu") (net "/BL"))
 (segment (start 110.3 122.7) (end 110.3 122.248101) (width 0.2) (layer "F.Cu") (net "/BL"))
 (segment (start 146.4 121.752314) (end 146.4 116.231372) (width 0.2) (layer "F.Cu") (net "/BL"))
 (segment (start 161.95 123.968) (end 161.95 117.884316) (width 0.2) (layer "F.Cu") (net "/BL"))
 (segment (start 162.75 123.968) (end 162.929899 123.968) (width 0.2) (layer "F.Cu") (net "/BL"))
 (segment (start 160.95 124.788101) (end 161.770101 123.968) (width 0.2) (layer "F.Cu") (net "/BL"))
 (segment (start 125.75 125.768) (end 125.75 125.947899) (width 0.2) (layer "F.Cu") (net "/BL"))
 (segment (start 161.95 117.884316) (end 147.2 103.134316) (width 0.2) (layer "F.Cu") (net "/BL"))
 (segment (start 141.95 125.947899) (end 141.95 124.788101) (width 0.2) (layer "F.Cu") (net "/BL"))
 (segment (start 110.3 122.248101) (end 117.548101 115) (width 0.2) (layer "F.Cu") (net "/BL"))
 (segment (start 129.133402 130.258) (end 127.186598 130.258) (width 0.2) (layer "F.Cu") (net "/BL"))
 (segment (start 147.2 122.083686) (end 144.622792 124.660894) (width 0.2) (layer "F.Cu") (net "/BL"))
 (segment (start 144.057107 124.095207) (end 146.4 121.752314) (width 0.2) (layer "F.Cu") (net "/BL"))
 (segment (start 144.6 108.165685) (end 144.6 103.002943) (width 0.2) (layer "F.Cu") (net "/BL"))
 (segment (start 143.929899 126.768) (end 142.770101 126.768) (width 0.2) (layer "F.Cu") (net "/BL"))
 (segment (start 126.976598 125.768) (end 125.75 125.768) (width 0.2) (layer "F.Cu") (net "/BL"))
 (segment (start 161.770101 123.968) (end 161.95 123.968) (width 0.2) (layer "F.Cu") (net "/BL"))
 (segment (start 142.770101 123.968) (end 143.929899 123.968) (width 0.2) (layer "F.Cu") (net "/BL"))
 (segment (start 125.81 128.881402) (end 125.81 126.934598) (width 0.2) (layer "F.Cu") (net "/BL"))
 (segment (start 145.6 109.183685) (end 145.6 107.334315) (width 0.2) (layer "F.Cu") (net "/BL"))
 (segment (start 130.51 126.934598) (end 130.51 128.881402) (width 0.2) (layer "F.Cu") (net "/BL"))
 (segment (start 146 103.300001) (end 145.9 103.400001) (width 0.2) (layer "F.Cu") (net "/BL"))
 (segment (start 144.75 125.947899) (end 143.929899 126.768) (width 0.2) (layer "F.Cu") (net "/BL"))
 (segment (start 162.75 117.552945) (end 162.75 123.968) (width 0.2) (layer "F.Cu") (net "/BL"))
 (segment (start 145.6 107.334315) (end 145.834315 107.1) (width 0.2) (layer "F.Cu") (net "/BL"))
 (segment (start 123.770101 123.968) (end 124.929899 123.968) (width 0.2) (layer "F.Cu") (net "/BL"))
 (segment (start 162.929899 123.968) (end 163.75 124.788101) (width 0.2) (layer "F.Cu") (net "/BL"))
 (segment (start 163.75 124.788101) (end 163.75 125.947899) (width 0.2) (layer "F.Cu") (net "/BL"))
 (segment (start 103.95 125.947899) (end 104.770101 126.768) (width 0.2) (layer "F.Cu") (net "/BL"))
 (segment (start 103.95 98.67) (end 103.95 125.947899) (width 0.2) (layer "F.Cu") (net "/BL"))
 (segment (start 145.665685 105.4) (end 145.4 105.4) (width 0.2) (layer "F.Cu") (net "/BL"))
 (segment (start 102 96.72) (end 103.95 98.67) (width 0.2) (layer "F.Cu") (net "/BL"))
 (segment (start 102 96.72) (end 104.35 99.07) (width 0.2) (layer "B.Cu") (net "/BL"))
 (segment (start 131.1305 116.46) (end 129.8305 115.16) (width 0.2) (layer "B.Cu") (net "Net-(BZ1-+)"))
 (segment (start 170.4 102.3) (end 156.24 116.46) (width 0.2) (layer "B.Cu") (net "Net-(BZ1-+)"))
 (segment (start 156.24 116.46) (end 131.1305 116.46) (width 0.2) (layer "B.Cu") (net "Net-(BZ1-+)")))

